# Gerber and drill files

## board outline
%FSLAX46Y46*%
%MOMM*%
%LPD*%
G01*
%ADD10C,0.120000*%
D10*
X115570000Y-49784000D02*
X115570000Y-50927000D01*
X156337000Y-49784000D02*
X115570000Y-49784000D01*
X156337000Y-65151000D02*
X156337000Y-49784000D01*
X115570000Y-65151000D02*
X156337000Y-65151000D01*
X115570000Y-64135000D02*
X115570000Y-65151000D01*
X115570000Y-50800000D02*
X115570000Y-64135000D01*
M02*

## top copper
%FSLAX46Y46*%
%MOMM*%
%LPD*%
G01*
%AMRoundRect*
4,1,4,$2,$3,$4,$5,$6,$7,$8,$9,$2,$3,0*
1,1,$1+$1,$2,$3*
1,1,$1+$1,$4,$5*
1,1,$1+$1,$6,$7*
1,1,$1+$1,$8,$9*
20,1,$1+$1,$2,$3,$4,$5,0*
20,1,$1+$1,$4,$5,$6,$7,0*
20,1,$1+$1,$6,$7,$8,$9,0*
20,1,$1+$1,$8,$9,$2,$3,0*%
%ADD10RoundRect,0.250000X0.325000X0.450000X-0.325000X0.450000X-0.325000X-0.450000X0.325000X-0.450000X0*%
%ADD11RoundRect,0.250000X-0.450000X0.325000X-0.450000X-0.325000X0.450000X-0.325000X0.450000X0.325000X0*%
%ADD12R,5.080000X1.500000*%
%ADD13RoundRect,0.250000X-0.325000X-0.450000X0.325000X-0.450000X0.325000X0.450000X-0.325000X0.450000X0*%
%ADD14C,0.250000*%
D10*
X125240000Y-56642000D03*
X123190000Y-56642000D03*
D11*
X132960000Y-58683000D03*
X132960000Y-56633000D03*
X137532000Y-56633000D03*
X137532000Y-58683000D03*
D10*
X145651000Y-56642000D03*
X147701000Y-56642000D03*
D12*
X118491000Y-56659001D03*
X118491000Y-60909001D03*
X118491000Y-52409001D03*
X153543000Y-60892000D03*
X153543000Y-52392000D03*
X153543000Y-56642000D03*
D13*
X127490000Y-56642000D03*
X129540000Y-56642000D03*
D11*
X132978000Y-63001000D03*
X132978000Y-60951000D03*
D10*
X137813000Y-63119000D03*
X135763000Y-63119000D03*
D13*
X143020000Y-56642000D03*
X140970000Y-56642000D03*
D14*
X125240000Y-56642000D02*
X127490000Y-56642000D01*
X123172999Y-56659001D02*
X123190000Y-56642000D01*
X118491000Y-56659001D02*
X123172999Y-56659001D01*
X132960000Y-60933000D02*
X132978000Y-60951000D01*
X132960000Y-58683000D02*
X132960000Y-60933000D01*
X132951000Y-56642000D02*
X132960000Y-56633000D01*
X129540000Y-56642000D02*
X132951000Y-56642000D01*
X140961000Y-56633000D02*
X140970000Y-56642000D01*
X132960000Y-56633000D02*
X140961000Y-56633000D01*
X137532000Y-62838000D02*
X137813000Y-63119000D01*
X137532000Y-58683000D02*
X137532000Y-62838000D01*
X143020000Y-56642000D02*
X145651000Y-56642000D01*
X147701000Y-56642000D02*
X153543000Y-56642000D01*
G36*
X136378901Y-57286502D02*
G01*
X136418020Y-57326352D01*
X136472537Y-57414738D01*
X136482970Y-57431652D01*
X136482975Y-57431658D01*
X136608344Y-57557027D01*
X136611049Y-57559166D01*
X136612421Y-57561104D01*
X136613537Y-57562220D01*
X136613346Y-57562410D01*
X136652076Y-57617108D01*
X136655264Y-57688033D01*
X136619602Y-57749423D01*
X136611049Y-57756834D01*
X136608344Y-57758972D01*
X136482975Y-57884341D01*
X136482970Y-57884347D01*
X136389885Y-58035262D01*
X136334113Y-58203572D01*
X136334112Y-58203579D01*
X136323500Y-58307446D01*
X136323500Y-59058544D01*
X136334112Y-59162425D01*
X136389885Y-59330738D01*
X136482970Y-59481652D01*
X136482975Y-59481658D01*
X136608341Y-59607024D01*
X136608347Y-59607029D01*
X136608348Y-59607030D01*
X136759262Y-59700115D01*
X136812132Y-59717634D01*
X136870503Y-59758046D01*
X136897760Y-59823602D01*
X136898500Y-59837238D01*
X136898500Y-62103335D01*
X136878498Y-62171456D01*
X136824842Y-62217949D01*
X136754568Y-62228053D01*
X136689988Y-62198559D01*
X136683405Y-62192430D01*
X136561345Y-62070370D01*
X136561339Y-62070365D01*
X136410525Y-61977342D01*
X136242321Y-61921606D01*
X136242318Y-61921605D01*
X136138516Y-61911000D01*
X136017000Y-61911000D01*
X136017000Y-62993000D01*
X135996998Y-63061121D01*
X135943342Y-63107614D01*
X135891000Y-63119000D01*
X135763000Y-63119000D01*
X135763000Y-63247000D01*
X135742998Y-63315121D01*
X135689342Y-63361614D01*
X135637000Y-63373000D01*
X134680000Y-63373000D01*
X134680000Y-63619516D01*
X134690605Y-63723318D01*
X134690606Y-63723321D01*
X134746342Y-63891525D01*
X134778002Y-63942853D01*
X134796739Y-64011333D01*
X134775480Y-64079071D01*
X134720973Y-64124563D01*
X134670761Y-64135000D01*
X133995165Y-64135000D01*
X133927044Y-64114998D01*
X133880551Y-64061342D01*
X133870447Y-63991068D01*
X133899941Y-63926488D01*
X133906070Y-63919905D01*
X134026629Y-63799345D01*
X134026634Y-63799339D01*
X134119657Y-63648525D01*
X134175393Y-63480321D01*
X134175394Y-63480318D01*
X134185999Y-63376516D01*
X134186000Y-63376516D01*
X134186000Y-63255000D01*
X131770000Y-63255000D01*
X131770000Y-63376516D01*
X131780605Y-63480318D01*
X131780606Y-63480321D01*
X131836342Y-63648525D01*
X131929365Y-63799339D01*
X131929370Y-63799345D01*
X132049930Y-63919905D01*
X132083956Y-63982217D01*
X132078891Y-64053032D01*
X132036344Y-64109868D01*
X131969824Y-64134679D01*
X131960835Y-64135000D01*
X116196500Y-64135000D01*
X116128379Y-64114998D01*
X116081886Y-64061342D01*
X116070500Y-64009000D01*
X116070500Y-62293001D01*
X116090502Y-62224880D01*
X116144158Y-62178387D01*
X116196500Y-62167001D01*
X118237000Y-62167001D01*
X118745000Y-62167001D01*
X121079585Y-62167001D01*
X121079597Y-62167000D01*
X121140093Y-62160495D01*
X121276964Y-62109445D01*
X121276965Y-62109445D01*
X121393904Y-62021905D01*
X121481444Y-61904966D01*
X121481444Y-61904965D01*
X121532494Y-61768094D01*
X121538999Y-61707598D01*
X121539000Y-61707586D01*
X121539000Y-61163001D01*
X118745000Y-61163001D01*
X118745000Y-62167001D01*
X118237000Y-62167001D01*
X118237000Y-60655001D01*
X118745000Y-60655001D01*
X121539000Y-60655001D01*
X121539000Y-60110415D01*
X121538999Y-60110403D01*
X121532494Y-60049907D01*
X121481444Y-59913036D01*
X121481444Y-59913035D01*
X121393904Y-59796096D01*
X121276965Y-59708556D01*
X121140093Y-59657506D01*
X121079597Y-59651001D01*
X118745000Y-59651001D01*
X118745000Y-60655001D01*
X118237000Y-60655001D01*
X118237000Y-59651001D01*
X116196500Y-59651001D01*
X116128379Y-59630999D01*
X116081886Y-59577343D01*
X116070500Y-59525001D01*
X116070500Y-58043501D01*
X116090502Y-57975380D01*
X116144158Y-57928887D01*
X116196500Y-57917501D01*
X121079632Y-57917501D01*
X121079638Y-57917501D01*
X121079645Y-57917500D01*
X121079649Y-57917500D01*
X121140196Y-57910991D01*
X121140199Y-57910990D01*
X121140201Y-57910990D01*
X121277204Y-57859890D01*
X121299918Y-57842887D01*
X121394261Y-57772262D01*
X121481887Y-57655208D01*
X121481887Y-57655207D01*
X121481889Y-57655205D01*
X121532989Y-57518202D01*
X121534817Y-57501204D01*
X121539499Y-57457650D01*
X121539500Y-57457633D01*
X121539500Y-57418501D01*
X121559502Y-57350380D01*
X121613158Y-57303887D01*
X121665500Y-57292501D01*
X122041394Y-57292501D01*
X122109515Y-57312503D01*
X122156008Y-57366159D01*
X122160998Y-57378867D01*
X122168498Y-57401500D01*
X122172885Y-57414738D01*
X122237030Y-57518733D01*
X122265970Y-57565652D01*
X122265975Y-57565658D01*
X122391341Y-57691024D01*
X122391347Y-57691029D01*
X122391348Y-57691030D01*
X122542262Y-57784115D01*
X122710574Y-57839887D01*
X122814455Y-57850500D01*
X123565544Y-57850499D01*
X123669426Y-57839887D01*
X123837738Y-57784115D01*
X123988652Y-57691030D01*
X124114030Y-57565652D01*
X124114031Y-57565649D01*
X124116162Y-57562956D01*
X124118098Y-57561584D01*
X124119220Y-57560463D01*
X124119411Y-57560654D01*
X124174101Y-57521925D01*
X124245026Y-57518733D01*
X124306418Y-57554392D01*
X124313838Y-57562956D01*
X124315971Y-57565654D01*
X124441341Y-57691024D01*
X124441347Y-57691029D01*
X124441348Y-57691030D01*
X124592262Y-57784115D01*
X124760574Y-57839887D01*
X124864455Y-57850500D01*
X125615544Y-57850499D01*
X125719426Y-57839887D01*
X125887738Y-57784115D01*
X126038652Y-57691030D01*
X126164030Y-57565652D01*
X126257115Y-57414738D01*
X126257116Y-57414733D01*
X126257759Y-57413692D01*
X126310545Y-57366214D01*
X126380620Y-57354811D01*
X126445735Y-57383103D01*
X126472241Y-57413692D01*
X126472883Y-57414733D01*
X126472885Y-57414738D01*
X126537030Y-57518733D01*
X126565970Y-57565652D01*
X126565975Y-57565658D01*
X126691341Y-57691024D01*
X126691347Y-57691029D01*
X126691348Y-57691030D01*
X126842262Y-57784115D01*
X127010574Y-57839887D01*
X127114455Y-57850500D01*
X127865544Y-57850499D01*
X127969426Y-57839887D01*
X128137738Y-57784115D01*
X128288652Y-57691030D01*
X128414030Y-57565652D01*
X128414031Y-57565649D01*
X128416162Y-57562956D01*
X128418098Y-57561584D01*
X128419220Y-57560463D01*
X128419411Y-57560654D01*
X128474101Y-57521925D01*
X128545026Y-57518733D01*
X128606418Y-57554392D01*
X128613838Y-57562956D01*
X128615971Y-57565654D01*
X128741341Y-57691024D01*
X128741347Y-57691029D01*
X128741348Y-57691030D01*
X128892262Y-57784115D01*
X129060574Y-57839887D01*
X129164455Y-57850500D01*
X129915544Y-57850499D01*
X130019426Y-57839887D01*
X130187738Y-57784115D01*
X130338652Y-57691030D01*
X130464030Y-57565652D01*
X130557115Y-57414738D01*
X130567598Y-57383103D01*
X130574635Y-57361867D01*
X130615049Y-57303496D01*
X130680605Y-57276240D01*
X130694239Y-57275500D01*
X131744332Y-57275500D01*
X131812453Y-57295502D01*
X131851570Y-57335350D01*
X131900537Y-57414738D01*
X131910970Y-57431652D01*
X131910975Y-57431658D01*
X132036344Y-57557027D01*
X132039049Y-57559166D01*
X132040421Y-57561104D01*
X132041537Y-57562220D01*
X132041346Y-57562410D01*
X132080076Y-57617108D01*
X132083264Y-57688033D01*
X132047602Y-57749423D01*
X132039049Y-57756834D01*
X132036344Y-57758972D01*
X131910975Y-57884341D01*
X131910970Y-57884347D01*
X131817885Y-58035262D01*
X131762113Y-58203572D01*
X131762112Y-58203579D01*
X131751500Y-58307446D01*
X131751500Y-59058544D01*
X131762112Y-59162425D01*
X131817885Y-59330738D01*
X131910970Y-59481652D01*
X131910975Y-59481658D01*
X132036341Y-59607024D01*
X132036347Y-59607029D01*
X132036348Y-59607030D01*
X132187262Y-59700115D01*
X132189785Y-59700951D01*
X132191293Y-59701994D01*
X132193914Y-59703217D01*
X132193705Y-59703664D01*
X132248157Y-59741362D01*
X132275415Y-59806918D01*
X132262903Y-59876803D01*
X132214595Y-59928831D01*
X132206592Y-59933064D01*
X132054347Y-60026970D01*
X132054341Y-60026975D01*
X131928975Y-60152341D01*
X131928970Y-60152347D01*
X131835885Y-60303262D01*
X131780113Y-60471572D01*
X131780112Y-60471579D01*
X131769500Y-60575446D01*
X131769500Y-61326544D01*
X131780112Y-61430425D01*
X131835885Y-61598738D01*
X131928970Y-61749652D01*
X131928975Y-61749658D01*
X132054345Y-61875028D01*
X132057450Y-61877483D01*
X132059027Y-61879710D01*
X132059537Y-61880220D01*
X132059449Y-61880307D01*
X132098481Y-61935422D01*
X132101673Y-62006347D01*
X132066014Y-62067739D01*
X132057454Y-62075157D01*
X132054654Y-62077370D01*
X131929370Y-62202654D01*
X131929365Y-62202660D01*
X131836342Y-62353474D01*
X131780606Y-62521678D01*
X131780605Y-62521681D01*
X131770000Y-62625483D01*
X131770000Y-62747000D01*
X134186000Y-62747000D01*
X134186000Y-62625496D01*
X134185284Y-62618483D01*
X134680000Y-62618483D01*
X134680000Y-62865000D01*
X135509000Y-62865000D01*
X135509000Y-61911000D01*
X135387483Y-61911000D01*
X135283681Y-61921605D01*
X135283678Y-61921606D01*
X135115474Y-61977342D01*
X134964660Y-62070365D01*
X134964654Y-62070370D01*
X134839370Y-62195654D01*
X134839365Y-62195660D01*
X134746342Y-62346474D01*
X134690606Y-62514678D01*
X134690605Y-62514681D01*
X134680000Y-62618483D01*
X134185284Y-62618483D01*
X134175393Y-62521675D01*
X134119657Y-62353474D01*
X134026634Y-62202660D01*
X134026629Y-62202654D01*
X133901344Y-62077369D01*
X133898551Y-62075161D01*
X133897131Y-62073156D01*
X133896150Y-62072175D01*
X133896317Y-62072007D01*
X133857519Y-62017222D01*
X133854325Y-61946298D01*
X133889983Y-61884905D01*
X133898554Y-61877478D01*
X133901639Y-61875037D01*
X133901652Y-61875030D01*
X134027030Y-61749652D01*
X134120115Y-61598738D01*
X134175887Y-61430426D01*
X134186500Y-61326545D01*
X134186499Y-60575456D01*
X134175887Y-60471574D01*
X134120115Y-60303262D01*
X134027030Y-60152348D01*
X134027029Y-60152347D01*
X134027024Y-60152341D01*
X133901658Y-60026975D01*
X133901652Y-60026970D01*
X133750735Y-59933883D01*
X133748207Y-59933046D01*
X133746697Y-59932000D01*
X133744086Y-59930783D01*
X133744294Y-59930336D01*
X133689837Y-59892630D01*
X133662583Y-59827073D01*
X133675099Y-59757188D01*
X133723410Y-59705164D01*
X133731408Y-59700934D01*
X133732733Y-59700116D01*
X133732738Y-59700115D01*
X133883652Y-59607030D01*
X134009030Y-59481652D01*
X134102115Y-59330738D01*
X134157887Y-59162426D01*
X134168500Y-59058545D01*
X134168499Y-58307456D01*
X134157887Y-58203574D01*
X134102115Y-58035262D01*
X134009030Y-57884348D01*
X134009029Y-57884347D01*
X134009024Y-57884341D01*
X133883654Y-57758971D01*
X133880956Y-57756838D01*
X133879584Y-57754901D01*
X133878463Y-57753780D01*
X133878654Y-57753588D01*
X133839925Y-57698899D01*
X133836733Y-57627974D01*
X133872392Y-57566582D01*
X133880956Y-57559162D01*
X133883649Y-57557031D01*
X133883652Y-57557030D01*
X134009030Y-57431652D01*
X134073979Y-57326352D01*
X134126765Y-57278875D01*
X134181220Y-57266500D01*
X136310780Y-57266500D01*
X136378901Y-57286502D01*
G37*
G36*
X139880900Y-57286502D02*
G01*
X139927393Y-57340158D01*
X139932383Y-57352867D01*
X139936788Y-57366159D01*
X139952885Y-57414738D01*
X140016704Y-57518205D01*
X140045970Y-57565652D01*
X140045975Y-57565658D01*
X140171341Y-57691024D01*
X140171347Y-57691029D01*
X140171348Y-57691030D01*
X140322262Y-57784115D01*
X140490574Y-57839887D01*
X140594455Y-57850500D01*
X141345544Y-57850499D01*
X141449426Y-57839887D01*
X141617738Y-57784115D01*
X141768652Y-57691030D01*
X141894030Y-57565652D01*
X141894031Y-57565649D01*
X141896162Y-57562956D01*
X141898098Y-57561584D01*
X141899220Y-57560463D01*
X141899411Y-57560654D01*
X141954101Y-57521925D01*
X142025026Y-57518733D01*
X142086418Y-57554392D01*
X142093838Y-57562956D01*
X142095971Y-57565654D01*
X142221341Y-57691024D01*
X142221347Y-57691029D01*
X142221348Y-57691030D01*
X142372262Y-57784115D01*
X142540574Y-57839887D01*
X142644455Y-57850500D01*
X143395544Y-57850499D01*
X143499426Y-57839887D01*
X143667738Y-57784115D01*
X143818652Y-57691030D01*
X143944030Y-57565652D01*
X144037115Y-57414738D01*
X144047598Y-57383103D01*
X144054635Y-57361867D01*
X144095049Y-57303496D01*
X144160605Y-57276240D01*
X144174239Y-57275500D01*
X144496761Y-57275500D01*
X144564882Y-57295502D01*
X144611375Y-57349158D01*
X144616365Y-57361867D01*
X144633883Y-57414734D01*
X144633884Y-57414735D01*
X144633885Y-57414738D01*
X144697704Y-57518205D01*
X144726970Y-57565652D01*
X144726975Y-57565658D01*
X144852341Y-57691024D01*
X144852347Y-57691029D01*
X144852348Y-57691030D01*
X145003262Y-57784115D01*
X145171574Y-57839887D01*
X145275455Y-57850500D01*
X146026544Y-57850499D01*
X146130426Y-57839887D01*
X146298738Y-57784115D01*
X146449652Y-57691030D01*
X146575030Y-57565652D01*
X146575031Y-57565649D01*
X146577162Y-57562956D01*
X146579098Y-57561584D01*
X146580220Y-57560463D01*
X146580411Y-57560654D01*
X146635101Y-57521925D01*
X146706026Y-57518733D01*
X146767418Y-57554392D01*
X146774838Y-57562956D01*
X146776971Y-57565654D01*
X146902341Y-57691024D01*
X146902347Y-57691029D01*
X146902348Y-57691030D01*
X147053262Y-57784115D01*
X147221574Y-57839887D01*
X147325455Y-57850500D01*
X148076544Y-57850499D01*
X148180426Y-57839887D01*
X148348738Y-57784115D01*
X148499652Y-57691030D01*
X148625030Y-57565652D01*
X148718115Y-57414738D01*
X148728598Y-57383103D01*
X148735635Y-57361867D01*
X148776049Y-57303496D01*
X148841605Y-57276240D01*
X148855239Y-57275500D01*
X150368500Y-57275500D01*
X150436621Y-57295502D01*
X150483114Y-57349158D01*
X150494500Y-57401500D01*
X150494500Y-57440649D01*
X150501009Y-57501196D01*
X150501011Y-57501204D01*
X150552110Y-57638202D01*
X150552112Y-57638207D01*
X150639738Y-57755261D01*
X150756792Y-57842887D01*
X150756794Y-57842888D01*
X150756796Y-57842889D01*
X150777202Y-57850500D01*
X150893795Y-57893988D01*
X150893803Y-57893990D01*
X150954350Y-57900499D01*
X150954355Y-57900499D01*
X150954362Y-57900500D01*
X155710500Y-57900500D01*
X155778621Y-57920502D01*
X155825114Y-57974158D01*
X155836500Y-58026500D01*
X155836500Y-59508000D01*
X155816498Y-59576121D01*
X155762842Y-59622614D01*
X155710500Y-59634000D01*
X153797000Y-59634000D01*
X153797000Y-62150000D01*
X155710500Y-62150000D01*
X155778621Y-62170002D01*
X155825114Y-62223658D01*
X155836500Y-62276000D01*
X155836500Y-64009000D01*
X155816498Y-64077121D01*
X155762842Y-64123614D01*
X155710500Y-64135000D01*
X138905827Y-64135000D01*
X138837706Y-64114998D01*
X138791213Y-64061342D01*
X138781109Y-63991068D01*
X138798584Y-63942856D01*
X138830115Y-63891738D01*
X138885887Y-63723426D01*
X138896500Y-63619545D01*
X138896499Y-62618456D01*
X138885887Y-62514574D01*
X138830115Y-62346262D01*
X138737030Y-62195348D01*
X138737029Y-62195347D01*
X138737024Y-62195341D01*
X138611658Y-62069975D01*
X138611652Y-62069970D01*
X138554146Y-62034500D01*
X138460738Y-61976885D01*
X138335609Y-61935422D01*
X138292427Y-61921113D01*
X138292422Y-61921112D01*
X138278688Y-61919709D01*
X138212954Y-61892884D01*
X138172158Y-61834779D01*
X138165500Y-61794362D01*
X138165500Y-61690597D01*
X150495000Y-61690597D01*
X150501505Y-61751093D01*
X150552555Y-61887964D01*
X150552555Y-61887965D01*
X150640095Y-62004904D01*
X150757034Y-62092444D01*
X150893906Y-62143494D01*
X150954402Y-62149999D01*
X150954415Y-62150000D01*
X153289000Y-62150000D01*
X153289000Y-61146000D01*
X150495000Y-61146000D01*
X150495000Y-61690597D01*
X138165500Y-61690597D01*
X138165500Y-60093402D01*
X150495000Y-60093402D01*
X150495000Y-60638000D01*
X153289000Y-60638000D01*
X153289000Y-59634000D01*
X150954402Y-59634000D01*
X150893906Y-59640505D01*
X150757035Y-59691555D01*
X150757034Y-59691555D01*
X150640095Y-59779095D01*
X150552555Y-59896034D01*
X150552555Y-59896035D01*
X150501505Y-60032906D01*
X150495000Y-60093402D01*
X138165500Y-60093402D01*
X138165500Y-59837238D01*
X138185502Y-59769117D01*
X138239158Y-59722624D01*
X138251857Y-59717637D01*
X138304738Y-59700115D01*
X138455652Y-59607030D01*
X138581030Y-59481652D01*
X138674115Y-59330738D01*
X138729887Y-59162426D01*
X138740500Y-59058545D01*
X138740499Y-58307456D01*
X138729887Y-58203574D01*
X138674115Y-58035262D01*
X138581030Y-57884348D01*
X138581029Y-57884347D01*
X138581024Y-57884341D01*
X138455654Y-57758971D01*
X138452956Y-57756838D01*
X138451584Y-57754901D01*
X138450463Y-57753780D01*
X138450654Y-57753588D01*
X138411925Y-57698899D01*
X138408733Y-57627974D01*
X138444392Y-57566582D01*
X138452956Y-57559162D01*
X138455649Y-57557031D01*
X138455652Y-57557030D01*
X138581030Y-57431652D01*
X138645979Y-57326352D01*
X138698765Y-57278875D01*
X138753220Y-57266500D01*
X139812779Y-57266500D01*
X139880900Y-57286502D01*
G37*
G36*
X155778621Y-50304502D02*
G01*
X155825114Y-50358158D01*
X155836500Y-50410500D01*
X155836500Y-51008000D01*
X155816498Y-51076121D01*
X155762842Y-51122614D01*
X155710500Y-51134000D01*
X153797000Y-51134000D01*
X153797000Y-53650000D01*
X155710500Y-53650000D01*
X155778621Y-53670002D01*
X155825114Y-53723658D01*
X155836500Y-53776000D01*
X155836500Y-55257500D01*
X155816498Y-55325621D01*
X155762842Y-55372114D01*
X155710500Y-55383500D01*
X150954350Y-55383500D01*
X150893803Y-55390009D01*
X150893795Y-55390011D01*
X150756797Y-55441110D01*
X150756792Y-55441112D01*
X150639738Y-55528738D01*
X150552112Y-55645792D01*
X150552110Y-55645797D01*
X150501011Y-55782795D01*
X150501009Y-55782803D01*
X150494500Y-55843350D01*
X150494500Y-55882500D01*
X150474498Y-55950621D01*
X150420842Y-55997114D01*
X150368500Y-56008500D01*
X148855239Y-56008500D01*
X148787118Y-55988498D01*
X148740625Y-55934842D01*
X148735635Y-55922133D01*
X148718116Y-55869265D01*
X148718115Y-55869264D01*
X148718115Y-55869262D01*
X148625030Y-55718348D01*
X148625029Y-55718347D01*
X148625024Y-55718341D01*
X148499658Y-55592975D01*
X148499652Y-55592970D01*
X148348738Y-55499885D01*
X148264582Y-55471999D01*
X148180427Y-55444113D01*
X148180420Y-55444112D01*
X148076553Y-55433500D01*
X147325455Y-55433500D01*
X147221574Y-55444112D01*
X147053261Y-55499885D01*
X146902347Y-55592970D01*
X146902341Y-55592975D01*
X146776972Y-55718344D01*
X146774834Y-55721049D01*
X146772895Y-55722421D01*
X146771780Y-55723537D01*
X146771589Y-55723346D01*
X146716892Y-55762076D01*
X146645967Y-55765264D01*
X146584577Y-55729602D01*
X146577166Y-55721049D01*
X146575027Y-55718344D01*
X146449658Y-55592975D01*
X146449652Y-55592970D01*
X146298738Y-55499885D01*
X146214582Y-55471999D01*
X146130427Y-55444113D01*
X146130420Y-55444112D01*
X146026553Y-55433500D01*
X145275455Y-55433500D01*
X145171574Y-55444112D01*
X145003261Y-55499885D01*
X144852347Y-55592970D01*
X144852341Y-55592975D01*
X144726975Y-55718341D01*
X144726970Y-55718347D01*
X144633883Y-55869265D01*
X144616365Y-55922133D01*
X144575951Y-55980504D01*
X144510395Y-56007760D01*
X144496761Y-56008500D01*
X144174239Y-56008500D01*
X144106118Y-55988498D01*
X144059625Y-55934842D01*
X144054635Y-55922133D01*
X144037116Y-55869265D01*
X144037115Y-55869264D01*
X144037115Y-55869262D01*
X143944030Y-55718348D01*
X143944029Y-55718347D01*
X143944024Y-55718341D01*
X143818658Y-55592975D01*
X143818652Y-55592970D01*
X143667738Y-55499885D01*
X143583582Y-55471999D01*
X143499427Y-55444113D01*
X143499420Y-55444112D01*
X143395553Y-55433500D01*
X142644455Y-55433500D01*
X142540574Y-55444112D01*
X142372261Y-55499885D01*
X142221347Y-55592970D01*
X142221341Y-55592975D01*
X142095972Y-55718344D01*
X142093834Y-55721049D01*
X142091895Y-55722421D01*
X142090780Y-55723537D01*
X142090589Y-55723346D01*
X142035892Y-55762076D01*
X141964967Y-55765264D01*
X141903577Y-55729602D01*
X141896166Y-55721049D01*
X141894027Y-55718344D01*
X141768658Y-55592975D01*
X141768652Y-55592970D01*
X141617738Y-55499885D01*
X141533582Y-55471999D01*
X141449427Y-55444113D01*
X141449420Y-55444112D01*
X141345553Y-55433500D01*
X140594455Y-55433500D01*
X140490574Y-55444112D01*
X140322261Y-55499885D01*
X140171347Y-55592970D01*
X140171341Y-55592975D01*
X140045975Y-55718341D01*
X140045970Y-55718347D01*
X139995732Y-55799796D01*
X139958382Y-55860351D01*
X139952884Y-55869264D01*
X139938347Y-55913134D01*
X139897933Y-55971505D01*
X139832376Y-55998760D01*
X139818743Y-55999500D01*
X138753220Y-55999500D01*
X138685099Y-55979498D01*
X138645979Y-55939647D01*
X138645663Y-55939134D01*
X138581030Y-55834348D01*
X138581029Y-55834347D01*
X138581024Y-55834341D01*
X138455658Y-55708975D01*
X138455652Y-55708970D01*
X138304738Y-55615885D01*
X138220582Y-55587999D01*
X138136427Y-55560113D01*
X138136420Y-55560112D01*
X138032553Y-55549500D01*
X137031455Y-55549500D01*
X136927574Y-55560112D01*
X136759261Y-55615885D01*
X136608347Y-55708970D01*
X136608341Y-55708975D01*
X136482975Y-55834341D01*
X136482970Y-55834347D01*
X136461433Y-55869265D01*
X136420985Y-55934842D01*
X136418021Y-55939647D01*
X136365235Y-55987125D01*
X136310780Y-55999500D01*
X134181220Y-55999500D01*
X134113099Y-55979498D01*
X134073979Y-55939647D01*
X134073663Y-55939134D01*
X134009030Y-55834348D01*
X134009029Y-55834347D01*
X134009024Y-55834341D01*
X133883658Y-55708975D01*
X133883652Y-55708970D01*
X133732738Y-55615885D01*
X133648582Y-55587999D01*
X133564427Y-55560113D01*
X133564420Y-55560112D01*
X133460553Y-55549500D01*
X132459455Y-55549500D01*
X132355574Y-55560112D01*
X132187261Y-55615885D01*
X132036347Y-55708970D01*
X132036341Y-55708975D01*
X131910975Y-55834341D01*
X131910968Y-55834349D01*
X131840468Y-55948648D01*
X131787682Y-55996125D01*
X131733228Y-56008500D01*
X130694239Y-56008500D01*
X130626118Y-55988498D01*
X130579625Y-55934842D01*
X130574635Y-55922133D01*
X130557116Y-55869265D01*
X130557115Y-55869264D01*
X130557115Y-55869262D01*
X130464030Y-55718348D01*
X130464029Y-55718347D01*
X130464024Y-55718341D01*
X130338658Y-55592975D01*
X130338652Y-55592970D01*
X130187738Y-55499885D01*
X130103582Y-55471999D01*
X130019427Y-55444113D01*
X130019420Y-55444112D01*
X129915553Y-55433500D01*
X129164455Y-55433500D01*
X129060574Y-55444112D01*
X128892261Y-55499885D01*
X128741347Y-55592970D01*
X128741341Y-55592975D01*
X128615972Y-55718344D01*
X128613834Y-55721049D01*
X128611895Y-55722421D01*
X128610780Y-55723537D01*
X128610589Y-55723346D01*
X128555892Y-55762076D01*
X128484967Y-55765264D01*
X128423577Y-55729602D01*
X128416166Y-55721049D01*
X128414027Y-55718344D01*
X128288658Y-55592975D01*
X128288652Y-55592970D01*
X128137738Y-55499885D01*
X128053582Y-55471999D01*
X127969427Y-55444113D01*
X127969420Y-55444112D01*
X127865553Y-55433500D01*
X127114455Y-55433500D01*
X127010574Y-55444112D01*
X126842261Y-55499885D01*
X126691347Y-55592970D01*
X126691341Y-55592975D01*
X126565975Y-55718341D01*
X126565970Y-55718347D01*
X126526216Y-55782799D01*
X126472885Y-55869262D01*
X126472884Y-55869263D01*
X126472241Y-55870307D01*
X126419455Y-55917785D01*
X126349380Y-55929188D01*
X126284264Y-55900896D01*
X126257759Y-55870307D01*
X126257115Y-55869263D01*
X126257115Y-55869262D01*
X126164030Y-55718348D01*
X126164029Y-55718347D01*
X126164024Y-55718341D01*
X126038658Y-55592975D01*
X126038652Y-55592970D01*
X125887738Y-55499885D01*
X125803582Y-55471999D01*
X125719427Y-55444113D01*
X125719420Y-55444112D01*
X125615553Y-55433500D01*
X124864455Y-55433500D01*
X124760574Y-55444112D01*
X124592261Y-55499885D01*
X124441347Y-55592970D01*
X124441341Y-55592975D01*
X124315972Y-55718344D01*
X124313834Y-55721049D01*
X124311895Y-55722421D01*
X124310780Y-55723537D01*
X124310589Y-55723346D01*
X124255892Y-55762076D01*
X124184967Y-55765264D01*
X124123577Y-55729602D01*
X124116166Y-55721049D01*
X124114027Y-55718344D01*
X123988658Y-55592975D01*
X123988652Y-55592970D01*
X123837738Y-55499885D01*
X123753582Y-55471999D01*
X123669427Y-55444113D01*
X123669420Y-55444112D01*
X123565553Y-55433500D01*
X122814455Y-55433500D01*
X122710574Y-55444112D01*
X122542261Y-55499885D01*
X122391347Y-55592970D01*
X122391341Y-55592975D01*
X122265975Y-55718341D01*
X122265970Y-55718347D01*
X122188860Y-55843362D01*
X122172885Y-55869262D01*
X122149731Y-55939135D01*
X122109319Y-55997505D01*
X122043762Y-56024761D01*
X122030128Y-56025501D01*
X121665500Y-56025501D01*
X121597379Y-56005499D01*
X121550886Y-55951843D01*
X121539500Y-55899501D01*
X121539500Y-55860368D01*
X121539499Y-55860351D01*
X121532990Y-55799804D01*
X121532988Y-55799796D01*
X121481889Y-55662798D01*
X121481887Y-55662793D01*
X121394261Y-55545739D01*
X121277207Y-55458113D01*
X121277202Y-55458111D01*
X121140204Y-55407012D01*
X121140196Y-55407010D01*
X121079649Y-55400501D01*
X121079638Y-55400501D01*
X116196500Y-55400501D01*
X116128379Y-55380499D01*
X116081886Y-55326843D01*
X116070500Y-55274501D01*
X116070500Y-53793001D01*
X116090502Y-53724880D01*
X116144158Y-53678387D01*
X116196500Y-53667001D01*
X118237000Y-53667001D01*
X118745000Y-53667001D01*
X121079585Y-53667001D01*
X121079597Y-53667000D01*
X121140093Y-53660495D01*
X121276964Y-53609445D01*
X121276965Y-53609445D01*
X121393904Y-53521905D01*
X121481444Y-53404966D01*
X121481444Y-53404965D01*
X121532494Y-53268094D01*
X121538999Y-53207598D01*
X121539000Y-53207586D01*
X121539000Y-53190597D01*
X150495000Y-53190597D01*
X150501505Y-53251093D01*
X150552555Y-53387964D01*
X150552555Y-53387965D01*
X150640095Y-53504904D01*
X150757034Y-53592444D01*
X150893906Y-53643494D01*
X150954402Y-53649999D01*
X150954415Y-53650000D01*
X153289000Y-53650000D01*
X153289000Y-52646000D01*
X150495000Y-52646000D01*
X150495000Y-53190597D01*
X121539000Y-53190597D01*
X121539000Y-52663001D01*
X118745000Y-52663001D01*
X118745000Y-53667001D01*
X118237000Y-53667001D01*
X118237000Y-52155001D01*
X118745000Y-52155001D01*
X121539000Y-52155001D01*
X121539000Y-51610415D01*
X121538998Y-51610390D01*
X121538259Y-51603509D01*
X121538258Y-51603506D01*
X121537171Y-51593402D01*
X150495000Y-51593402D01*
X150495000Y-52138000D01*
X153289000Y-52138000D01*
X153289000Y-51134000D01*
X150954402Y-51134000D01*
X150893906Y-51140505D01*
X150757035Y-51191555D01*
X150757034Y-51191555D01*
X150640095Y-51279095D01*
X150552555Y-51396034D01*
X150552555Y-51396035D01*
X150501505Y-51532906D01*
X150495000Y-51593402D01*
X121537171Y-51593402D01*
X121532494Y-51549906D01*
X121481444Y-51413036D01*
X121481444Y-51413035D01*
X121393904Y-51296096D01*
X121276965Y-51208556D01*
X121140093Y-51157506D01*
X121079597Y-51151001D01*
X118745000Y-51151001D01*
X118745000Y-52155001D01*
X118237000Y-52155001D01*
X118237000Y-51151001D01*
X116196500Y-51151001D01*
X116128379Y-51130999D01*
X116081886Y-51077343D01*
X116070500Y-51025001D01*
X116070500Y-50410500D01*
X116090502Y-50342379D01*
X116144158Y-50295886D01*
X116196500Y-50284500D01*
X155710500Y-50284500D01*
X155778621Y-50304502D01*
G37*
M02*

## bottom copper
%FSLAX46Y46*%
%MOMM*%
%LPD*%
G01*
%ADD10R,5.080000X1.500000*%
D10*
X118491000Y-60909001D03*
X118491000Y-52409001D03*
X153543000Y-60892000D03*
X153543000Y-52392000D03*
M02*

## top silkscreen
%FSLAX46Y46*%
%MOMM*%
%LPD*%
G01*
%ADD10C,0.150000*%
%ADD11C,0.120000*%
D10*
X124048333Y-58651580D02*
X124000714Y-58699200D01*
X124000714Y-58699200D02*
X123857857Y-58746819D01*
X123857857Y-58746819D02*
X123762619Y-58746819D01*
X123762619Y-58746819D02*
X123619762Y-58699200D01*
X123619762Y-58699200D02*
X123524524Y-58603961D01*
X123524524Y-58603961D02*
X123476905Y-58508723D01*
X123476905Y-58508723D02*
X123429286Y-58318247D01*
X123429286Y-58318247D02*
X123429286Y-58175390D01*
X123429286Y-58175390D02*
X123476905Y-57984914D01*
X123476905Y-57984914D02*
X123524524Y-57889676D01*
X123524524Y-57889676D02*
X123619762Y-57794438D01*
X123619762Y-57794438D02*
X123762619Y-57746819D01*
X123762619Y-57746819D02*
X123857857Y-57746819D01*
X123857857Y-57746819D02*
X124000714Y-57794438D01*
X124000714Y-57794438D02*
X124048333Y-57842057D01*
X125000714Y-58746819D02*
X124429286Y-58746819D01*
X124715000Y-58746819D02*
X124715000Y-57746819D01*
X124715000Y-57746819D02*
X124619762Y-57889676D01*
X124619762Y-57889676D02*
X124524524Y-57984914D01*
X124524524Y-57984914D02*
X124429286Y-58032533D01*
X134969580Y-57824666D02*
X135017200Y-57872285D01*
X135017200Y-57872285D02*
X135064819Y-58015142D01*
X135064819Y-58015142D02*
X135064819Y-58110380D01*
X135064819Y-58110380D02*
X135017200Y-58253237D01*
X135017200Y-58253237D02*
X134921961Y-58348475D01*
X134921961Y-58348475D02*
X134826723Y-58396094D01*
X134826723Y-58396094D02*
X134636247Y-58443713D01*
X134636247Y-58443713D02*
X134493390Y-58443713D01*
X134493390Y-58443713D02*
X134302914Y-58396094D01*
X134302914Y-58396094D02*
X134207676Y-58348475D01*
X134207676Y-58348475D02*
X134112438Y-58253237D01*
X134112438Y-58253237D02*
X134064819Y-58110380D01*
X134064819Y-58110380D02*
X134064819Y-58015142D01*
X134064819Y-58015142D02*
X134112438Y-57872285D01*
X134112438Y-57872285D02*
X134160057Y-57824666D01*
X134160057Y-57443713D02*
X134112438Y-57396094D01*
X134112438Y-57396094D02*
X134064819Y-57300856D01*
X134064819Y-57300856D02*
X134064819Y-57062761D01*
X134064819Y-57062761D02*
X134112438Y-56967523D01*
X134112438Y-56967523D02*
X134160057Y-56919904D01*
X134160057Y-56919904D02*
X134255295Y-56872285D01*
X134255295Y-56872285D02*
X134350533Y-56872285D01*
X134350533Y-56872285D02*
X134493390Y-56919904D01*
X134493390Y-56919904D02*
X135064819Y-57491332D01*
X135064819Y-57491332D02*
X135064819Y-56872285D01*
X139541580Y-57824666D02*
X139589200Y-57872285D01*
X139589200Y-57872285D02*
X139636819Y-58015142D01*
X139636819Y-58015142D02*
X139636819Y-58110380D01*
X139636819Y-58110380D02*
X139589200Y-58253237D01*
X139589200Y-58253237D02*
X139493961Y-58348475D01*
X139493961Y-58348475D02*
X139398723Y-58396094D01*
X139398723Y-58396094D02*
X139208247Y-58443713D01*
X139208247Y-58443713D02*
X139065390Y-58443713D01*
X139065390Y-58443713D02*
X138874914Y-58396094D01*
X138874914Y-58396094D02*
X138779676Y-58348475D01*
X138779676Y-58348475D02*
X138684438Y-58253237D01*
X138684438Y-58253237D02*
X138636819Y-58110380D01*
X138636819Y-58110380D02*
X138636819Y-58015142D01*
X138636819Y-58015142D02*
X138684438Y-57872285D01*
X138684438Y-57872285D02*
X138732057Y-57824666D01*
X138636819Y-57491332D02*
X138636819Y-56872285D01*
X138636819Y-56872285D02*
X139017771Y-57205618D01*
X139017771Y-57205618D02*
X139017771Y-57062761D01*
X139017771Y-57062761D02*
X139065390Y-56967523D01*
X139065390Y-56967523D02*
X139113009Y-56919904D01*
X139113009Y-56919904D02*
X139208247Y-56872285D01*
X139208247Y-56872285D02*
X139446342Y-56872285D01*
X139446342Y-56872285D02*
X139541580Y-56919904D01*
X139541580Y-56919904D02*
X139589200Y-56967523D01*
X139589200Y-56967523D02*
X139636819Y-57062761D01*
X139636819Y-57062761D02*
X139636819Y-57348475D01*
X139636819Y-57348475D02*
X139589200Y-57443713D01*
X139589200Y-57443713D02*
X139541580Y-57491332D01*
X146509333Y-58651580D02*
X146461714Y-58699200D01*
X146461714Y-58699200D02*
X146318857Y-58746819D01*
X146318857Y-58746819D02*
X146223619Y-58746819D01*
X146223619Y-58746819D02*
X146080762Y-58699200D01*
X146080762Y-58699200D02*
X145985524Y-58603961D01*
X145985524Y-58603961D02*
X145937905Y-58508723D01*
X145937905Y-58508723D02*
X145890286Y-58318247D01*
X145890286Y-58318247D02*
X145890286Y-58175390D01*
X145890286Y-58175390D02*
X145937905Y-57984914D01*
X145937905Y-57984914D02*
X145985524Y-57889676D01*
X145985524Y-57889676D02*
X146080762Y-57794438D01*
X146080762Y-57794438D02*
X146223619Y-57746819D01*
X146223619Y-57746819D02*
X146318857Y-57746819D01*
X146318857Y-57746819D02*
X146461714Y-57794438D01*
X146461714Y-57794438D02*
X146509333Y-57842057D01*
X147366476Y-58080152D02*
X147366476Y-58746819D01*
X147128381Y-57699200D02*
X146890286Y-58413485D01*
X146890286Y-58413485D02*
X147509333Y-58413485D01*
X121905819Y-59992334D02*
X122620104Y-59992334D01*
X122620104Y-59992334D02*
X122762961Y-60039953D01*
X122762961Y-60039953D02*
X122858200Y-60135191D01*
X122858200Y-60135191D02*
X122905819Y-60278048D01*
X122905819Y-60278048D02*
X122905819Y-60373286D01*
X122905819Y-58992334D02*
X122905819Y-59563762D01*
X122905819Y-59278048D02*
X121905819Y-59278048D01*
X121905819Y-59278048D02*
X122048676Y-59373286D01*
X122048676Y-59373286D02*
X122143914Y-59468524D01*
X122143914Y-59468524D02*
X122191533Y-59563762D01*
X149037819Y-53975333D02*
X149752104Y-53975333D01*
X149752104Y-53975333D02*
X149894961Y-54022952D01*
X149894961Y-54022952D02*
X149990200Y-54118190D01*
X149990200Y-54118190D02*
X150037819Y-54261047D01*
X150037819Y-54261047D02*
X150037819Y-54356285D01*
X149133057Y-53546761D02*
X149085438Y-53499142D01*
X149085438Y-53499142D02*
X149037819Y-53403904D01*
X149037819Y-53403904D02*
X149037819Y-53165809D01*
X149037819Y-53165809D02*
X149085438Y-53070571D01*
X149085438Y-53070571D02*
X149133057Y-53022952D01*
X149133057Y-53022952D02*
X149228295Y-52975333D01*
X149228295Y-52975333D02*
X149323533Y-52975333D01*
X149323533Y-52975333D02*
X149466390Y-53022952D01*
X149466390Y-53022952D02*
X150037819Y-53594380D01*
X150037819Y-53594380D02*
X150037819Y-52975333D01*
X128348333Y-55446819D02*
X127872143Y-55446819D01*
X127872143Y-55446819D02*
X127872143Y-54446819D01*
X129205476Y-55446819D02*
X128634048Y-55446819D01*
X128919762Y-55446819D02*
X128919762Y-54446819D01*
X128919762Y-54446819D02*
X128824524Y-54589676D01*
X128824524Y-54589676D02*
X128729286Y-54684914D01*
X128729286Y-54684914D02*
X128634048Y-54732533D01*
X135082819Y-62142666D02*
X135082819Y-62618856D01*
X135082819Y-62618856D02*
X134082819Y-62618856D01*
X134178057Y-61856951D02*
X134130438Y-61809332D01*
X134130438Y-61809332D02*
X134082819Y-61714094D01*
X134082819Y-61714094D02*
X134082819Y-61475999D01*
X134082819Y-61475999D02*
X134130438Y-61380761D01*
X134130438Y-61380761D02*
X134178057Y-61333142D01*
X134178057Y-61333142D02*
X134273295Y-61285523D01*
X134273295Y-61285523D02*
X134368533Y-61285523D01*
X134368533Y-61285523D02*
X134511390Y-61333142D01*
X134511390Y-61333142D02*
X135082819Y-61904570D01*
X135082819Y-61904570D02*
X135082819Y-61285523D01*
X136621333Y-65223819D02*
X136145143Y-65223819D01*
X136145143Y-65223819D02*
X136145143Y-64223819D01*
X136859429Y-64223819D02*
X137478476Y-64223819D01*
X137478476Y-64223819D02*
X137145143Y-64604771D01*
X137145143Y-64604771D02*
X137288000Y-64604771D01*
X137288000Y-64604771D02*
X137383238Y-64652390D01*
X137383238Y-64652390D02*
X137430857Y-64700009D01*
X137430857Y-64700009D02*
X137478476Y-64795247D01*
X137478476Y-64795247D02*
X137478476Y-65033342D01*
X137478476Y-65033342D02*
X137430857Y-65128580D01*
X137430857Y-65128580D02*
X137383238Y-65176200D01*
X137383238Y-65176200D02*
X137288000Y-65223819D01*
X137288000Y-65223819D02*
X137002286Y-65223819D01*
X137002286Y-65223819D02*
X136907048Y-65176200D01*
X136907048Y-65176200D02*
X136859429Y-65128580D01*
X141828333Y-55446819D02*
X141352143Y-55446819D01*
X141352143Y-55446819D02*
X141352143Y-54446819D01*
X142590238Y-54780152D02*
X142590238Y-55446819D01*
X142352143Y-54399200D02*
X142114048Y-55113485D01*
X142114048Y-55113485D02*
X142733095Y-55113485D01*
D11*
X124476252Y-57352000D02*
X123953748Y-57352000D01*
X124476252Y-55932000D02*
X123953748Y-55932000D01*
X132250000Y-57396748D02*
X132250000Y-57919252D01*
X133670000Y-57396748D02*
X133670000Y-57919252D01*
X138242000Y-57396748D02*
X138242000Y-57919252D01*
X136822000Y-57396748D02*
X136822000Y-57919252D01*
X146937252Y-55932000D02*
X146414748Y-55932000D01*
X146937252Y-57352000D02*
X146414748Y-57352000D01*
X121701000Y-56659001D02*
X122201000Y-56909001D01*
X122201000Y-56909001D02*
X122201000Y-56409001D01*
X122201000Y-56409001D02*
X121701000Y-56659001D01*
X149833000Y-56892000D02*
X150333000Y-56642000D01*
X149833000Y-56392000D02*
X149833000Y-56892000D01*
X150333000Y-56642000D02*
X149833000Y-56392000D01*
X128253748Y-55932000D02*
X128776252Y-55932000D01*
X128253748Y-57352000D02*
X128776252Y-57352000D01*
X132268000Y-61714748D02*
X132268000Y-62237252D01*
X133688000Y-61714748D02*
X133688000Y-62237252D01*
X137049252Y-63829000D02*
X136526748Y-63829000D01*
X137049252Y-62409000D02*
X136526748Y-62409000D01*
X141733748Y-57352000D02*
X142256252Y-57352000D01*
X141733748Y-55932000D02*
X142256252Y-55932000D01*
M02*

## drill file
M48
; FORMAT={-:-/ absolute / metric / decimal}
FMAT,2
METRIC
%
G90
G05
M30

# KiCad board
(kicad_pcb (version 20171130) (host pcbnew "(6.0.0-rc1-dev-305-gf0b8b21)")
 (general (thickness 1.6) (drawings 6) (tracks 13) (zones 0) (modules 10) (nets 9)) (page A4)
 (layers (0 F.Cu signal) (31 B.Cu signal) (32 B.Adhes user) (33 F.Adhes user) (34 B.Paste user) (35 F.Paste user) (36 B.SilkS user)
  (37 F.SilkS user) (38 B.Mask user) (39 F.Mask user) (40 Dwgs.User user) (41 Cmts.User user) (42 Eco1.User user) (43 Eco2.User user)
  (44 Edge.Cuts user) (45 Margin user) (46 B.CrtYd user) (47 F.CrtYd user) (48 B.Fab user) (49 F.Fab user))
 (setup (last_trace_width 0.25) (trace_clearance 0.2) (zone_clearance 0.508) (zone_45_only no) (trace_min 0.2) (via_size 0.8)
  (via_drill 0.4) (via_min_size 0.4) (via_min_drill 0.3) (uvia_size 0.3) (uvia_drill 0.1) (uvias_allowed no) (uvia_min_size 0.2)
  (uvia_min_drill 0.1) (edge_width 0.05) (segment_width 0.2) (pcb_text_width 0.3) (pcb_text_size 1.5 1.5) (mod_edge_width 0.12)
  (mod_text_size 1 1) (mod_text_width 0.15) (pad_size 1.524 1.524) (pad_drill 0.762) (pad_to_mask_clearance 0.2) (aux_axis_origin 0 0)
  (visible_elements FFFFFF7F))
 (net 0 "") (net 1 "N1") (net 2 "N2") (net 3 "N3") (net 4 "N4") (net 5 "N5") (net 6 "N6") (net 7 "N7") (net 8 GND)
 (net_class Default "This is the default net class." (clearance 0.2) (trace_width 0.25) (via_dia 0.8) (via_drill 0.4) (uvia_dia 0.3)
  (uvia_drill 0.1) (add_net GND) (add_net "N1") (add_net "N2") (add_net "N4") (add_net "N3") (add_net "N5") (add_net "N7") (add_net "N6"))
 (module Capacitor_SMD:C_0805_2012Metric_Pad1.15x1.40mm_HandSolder (layer F.Cu) (at 124.215 56.642 180)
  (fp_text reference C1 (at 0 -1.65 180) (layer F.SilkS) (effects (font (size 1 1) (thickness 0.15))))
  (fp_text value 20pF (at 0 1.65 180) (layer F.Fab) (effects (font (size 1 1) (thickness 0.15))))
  (fp_line (start -0.261252 -0.71) (end 0.261252 -0.71) (layer F.SilkS) (width 0.12))
  (fp_line (start -0.261252 0.71) (end 0.261252 0.71) (layer F.SilkS) (width 0.12))
  (pad 1 smd roundrect (at -1.025 0 180) (size 1.15 1.4) (layers F.Cu F.Paste F.Mask) (roundrect_rratio 0.217391) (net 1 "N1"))
  (pad 2 smd roundrect (at 1.025 0 180) (size 1.15 1.4) (layers F.Cu F.Paste F.Mask) (roundrect_rratio 0.217391) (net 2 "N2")))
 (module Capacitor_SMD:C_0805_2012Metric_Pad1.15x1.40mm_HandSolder (layer F.Cu) (at 132.96 57.658 270)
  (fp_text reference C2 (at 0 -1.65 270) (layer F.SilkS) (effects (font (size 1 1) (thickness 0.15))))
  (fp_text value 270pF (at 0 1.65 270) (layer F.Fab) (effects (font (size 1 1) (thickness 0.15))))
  (fp_line (start -0.261252 0.71) (end 0.261252 0.71) (layer F.SilkS) (width 0.12))
  (fp_line (start -0.261252 -0.71) (end 0.261252 -0.71) (layer F.SilkS) (width 0.12))
  (pad 2 smd roundrect (at 1.025 0 270) (size 1.15 1.4) (layers F.Cu F.Paste F.Mask) (roundrect_rratio 0.217391) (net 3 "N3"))
  (pad 1 smd roundrect (at -1.025 0 270) (size 1.15 1.4) (layers F.Cu F.Paste F.Mask) (roundrect_rratio 0.217391) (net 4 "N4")))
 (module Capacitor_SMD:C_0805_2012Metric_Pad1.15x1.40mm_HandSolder (layer F.Cu) (at 137.532 57.658 270)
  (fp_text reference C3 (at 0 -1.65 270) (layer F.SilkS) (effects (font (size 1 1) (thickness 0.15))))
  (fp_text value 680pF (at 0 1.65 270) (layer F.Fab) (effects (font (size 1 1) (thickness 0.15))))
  (fp_line (start -0.261252 -0.71) (end 0.261252 -0.71) (layer F.SilkS) (width 0.12))
  (fp_line (start -0.261252 0.71) (end 0.261252 0.71) (layer F.SilkS) (width 0.12))
  (pad 1 smd roundrect (at -1.025 0 270) (size 1.15 1.4) (layers F.Cu F.Paste F.Mask) (roundrect_rratio 0.217391) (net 4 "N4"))
  (pad 2 smd roundrect (at 1.025 0 270) (size 1.15 1.4) (layers F.Cu F.Paste F.Mask) (roundrect_rratio 0.217391) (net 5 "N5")))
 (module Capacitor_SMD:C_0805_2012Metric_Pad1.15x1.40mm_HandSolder (layer F.Cu) (at 146.676 56.642 180)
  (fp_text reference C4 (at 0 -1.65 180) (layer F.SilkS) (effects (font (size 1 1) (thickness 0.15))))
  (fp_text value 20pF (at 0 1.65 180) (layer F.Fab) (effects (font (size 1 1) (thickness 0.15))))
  (fp_line (start -0.261252 0.71) (end 0.261252 0.71) (layer F.SilkS) (width 0.12))
  (fp_line (start -0.261252 -0.71) (end 0.261252 -0.71) (layer F.SilkS) (width 0.12))
  (pad 2 smd roundrect (at 1.025 0 180) (size 1.15 1.4) (layers F.Cu F.Paste F.Mask) (roundrect_rratio 0.217391) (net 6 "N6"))
  (pad 1 smd roundrect (at -1.025 0 180) (size 1.15 1.4) (layers F.Cu F.Paste F.Mask) (roundrect_rratio 0.217391) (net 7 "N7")))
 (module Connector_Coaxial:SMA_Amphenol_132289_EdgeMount (layer F.Cu) (at 118.491 56.659001 180)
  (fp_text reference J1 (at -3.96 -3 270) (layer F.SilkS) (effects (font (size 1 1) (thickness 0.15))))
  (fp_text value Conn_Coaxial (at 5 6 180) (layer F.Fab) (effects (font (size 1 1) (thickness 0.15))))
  (fp_line (start -3.21 0) (end -3.71 -0.25) (layer F.SilkS) (width 0.12))
  (fp_line (start -3.71 -0.25) (end -3.71 0.25) (layer F.SilkS) (width 0.12))
  (fp_line (start -3.71 0.25) (end -3.21 0) (layer F.SilkS) (width 0.12))
  (pad 1 smd rect (at 0 0 270) (size 1.5 5.08) (layers F.Cu F.Paste F.Mask) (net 2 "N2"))
  (pad 2 smd rect (at 0 -4.25 270) (size 1.5 5.08) (layers F.Cu F.Paste F.Mask) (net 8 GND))
  (pad 2 smd rect (at 0 4.25 270) (size 1.5 5.08) (layers F.Cu F.Paste F.Mask) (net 8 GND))
  (pad 2 smd rect (at 0 -4.25 270) (size 1.5 5.08) (layers B.Cu B.Paste B.Mask) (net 8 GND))
  (pad 2 smd rect (at 0 4.25 270) (size 1.5 5.08) (layers B.Cu B.Paste B.Mask) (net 8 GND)))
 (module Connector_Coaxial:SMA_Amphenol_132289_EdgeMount (layer F.Cu) (at 153.543 56.642)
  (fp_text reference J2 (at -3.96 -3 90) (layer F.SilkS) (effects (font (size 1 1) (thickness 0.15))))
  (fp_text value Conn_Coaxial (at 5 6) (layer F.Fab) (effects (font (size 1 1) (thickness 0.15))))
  (fp_line (start -3.71 0.25) (end -3.21 0) (layer F.SilkS) (width 0.12))
  (fp_line (start -3.71 -0.25) (end -3.71 0.25) (layer F.SilkS) (width 0.12))
  (fp_line (start -3.21 0) (end -3.71 -0.25) (layer F.SilkS) (width 0.12))
  (pad 2 smd rect (at 0 4.25 90) (size 1.5 5.08) (layers B.Cu B.Paste B.Mask) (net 8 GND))
  (pad 2 smd rect (at 0 -4.25 90) (size 1.5 5.08) (layers B.Cu B.Paste B.Mask) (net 8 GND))
  (pad 2 smd rect (at 0 4.25 90) (size 1.5 5.08) (layers F.Cu F.Paste F.Mask) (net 8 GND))
  (pad 2 smd rect (at 0 -4.25 90) (size 1.5 5.08) (layers F.Cu F.Paste F.Mask) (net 8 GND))
  (pad 1 smd rect (at 0 0 90) (size 1.5 5.08) (layers F.Cu F.Paste F.Mask) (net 7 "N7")))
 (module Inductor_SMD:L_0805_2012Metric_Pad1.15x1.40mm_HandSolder (layer F.Cu) (at 128.515 56.642)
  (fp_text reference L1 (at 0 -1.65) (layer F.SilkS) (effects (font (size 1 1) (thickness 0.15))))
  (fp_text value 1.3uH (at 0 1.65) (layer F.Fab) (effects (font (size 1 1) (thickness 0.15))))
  (fp_line (start -0.261252 -0.71) (end 0.261252 -0.71) (layer F.SilkS) (width 0.12))
  (fp_line (start -0.261252 0.71) (end 0.261252 0.71) (layer F.SilkS) (width 0.12))
  (pad 1 smd roundrect (at -1.025 0) (size 1.15 1.4) (layers F.Cu F.Paste F.Mask) (roundrect_rratio 0.217391) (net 1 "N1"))
  (pad 2 smd roundrect (at 1.025 0) (size 1.15 1.4) (layers F.Cu F.Paste F.Mask) (roundrect_rratio 0.217391) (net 4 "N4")))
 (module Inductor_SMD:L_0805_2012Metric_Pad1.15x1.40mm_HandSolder (layer F.Cu) (at 132.978 61.976 270)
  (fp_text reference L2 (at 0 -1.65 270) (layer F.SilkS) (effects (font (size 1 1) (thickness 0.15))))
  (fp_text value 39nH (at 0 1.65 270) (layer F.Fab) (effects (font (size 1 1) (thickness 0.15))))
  (fp_line (start -0.261252 0.71) (end 0.261252 0.71) (layer F.SilkS) (width 0.12))
  (fp_line (start -0.261252 -0.71) (end 0.261252 -0.71) (layer F.SilkS) (width 0.12))
  (pad 2 smd roundrect (at 1.025 0 270) (size 1.15 1.4) (layers F.Cu F.Paste F.Mask) (roundrect_rratio 0.217391) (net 8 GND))
  (pad 1 smd roundrect (at -1.025 0 270) (size 1.15 1.4) (layers F.Cu F.Paste F.Mask) (roundrect_rratio 0.217391) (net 3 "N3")))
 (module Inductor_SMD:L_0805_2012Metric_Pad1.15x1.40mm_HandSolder (layer F.Cu) (at 136.788 63.119 180)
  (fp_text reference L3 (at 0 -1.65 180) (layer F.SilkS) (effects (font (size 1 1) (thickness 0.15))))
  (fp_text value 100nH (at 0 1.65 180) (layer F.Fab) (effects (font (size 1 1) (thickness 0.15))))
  (fp_line (start -0.261252 -0.71) (end 0.261252 -0.71) (layer F.SilkS) (width 0.12))
  (fp_line (start -0.261252 0.71) (end 0.261252 0.71) (layer F.SilkS) (width 0.12))
  (pad 1 smd roundrect (at -1.025 0 180) (size 1.15 1.4) (layers F.Cu F.Paste F.Mask) (roundrect_rratio 0.217391) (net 5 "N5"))
  (pad 2 smd roundrect (at 1.025 0 180) (size 1.15 1.4) (layers F.Cu F.Paste F.Mask) (roundrect_rratio 0.217391) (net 8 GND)))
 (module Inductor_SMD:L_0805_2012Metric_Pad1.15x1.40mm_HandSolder (layer F.Cu) (at 141.995 56.642)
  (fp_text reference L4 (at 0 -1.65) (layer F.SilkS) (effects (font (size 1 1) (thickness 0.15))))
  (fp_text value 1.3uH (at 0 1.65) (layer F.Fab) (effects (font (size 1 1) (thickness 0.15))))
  (fp_line (start -0.261252 0.71) (end 0.261252 0.71) (layer F.SilkS) (width 0.12))
  (fp_line (start -0.261252 -0.71) (end 0.261252 -0.71) (layer F.SilkS) (width 0.12))
  (pad 2 smd roundrect (at 1.025 0) (size 1.15 1.4) (layers F.Cu F.Paste F.Mask) (roundrect_rratio 0.217391) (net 6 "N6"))
  (pad 1 smd roundrect (at -1.025 0) (size 1.15 1.4) (layers F.Cu F.Paste F.Mask) (roundrect_rratio 0.217391) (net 4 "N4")))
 (gr_line (start 115.57 49.784) (end 115.57 50.927) (layer Edge.Cuts) (width 0.12))
 (gr_line (start 156.337 49.784) (end 115.57 49.784) (layer Edge.Cuts) (width 0.12))
 (gr_line (start 156.337 65.151) (end 156.337 49.784) (layer Edge.Cuts) (width 0.12))
 (gr_line (start 115.57 65.151) (end 156.337 65.151) (layer Edge.Cuts) (width 0.12))
 (gr_line (start 115.57 64.135) (end 115.57 65.151) (layer Edge.Cuts) (width 0.12))
 (gr_line (start 115.57 50.8) (end 115.57 64.135) (layer Edge.Cuts) (width 0.12))
 (segment (start 125.24 56.642) (end 127.49 56.642) (width 0.25) (layer F.Cu) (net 1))
 (segment (start 123.172999 56.659001) (end 123.19 56.642) (width 0.25) (layer F.Cu) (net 2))
 (segment (start 118.491 56.659001) (end 123.172999 56.659001) (width 0.25) (layer F.Cu) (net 2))
 (segment (start 132.96 60.933) (end 132.978 60.951) (width 0.25) (layer F.Cu) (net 3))
 (segment (start 132.96 58.683) (end 132.96 60.933) (width 0.25) (layer F.Cu) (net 3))
 (segment (start 132.951 56.642) (end 132.96 56.633) (width 0.25) (layer F.Cu) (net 4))
 (segment (start 129.54 56.642) (end 132.951 56.642) (width 0.25) (layer F.Cu) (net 4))
 (segment (start 140.961 56.633) (end 140.97 56.642) (width 0.25) (layer F.Cu) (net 4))
 (segment (start 132.96 56.633) (end 140.961 56.633) (width 0.25) (layer F.Cu) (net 4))
 (segment (start 137.532 62.838) (end 137.813 63.119) (width 0.25) (layer F.Cu) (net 5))
 (segment (start 137.532 58.683) (end 137.532 62.838) (width 0.25) (layer F.Cu) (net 5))
 (segment (start 143.02 56.642) (end 145.651 56.642) (width 0.25) (layer F.Cu) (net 6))
 (segment (start 147.701 56.642) (end 153.543 56.642) (width 0.25) (layer F.Cu) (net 7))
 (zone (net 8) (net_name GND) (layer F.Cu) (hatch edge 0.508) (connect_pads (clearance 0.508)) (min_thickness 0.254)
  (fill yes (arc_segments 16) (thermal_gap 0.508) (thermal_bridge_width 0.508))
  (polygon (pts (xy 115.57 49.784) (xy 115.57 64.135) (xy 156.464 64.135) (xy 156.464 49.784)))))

